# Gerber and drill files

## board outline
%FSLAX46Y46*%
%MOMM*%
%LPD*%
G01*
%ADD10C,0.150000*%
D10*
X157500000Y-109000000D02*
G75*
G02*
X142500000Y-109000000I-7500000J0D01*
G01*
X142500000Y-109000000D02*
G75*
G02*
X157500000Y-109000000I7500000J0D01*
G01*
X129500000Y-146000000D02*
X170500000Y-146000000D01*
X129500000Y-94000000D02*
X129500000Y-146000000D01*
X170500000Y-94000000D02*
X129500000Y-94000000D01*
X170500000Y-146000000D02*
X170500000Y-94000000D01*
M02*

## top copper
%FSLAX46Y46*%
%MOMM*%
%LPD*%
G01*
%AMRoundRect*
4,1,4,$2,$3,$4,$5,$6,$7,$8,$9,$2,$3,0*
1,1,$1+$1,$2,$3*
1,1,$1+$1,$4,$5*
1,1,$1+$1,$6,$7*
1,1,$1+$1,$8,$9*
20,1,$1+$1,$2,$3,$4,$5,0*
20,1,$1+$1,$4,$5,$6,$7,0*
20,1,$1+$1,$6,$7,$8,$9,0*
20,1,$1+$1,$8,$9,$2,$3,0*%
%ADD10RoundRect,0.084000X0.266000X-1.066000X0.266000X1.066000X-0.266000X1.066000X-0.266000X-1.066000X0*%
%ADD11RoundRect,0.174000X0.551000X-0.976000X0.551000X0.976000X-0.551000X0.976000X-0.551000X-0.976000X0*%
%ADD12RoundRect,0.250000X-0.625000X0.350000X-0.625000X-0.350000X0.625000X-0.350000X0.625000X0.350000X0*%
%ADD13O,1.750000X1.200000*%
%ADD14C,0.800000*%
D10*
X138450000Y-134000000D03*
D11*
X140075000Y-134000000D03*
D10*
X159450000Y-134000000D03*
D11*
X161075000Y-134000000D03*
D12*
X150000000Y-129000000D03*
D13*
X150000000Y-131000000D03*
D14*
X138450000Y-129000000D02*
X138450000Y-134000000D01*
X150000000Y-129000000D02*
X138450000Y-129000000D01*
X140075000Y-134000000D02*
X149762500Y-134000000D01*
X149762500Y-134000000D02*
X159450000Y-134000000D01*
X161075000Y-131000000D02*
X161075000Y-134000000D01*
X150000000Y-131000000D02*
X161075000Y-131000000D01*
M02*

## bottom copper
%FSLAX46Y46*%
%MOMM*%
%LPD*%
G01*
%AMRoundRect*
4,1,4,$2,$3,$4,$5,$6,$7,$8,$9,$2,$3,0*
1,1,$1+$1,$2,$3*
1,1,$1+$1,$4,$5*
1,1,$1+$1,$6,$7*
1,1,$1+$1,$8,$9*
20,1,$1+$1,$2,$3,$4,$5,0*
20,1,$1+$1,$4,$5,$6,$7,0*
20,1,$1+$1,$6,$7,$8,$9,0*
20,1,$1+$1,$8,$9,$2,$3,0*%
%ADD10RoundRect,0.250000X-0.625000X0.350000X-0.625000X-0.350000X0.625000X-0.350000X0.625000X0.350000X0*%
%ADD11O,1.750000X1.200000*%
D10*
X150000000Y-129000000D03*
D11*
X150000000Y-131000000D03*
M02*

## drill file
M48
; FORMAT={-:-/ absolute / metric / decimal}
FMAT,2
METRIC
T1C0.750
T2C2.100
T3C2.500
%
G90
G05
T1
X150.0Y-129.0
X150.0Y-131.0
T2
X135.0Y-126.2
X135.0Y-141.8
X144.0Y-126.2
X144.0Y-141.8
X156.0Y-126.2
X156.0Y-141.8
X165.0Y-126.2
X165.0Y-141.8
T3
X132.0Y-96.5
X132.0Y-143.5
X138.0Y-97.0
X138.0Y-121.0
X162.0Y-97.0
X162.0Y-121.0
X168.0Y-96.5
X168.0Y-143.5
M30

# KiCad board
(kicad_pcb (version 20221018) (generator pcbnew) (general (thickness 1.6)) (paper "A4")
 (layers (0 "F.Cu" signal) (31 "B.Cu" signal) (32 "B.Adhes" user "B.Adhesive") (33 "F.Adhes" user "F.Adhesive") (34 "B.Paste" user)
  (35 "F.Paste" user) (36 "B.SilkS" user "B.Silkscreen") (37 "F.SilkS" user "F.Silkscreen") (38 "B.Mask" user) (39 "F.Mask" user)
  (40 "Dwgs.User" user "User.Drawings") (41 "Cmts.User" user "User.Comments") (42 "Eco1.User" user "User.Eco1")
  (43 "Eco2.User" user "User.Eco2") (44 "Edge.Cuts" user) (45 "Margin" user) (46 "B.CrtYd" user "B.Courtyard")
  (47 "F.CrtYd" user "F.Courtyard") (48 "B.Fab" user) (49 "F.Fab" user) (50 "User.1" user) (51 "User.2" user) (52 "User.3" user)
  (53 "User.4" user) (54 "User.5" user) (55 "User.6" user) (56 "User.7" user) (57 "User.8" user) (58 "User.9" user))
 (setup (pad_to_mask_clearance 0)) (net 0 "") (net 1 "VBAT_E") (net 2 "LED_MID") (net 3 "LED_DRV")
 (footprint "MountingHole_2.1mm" (layer "F.Cu") (at 144 126.2)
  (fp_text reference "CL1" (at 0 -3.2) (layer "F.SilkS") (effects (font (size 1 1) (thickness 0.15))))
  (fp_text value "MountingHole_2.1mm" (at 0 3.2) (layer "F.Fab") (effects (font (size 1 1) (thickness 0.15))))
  (pad "" np_thru_hole circle (at 0 0) (size 2.1 2.1) (drill 2.1) (layers "*.Cu" "*.Mask")))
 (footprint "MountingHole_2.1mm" (layer "F.Cu") (at 135 126.2)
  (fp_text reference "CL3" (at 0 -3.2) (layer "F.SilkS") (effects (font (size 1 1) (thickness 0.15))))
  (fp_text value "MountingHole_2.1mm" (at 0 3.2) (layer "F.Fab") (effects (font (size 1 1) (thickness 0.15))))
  (pad "" np_thru_hole circle (at 0 0) (size 2.1 2.1) (drill 2.1) (layers "*.Cu" "*.Mask")))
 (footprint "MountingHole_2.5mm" (layer "F.Cu") (at 138 121)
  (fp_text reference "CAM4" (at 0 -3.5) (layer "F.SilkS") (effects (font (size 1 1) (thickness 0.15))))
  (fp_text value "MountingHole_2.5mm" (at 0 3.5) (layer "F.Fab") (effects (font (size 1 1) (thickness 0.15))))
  (pad "" np_thru_hole circle (at 0 0) (size 2.5 2.5) (drill 2.5) (layers "*.Cu" "*.Mask")))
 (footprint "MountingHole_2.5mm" (layer "F.Cu") (at 168 96.5)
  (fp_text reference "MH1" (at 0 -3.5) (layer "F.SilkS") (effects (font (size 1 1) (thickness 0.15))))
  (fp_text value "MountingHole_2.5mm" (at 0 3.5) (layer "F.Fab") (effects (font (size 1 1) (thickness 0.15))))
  (pad "" np_thru_hole circle (at 0 0) (size 2.5 2.5) (drill 2.5) (layers "*.Cu" "*.Mask")))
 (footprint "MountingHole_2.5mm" (layer "F.Cu") (at 132 96.5)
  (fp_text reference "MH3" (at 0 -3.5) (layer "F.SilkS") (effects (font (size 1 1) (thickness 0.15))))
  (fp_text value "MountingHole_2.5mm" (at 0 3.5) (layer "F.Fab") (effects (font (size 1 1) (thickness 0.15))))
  (pad "" np_thru_hole circle (at 0 0) (size 2.5 2.5) (drill 2.5) (layers "*.Cu" "*.Mask")))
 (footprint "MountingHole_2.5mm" (layer "F.Cu") (at 138 97)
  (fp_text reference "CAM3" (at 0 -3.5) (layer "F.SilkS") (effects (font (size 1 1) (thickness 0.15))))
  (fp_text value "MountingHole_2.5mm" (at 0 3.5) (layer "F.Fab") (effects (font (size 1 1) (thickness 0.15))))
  (pad "" np_thru_hole circle (at 0 0) (size 2.5 2.5) (drill 2.5) (layers "*.Cu" "*.Mask")))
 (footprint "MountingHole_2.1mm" (layer "F.Cu") (at 135 141.8)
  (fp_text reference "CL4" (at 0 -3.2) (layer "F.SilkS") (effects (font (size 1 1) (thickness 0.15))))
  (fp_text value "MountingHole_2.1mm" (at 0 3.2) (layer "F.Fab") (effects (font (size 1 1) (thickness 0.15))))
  (pad "" np_thru_hole circle (at 0 0) (size 2.1 2.1) (drill 2.1) (layers "*.Cu" "*.Mask")))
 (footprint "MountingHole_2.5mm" (layer "F.Cu") (at 168 143.5)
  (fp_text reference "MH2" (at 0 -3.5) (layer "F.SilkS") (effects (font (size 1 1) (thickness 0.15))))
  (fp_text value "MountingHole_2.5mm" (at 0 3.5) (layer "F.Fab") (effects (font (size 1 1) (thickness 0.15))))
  (pad "" np_thru_hole circle (at 0 0) (size 2.5 2.5) (drill 2.5) (layers "*.Cu" "*.Mask")))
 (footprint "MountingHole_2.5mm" (layer "F.Cu") (at 162 121)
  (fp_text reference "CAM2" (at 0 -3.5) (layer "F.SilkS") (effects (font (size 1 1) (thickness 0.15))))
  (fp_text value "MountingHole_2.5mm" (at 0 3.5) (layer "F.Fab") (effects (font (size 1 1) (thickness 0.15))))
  (pad "" np_thru_hole circle (at 0 0) (size 2.5 2.5) (drill 2.5) (layers "*.Cu" "*.Mask")))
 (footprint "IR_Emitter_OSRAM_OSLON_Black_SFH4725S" (layer "F.Cu") (at 139.5 134 90)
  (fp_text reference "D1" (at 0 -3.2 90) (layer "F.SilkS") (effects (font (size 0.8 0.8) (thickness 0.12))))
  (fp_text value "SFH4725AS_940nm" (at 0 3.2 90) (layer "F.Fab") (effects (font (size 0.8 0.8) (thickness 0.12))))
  (pad "1" smd roundrect (at 0 -1.05 90) (size 2.3 0.7) (layers "F.Cu" "F.Paste" "F.Mask") (roundrect_rratio 0.12) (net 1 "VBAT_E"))
  (pad "2" smd roundrect (at 0 0.575 90) (size 2.3 1.45) (layers "F.Cu" "F.Paste" "F.Mask") (roundrect_rratio 0.12) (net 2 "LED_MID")))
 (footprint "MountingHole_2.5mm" (layer "F.Cu") (at 132 143.5)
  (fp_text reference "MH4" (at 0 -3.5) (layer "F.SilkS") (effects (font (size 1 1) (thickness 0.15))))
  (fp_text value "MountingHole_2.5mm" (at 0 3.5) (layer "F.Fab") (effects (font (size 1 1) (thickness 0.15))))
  (pad "" np_thru_hole circle (at 0 0) (size 2.5 2.5) (drill 2.5) (layers "*.Cu" "*.Mask")))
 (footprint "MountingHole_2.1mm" (layer "F.Cu") (at 156 141.8)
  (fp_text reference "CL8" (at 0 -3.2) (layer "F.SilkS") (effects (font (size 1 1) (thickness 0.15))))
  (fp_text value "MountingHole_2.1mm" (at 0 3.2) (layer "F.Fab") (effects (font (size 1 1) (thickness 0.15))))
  (pad "" np_thru_hole circle (at 0 0) (size 2.1 2.1) (drill 2.1) (layers "*.Cu" "*.Mask")))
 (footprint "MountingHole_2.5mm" (layer "F.Cu") (at 162 97)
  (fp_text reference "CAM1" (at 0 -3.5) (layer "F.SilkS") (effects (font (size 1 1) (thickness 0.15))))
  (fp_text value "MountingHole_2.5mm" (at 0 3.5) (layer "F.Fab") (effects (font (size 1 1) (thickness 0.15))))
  (pad "" np_thru_hole circle (at 0 0) (size 2.5 2.5) (drill 2.5) (layers "*.Cu" "*.Mask")))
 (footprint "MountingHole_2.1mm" (layer "F.Cu") (at 165 126.2)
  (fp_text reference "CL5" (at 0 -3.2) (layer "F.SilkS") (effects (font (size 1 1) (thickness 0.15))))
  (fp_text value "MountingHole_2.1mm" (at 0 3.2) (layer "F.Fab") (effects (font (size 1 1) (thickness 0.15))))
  (pad "" np_thru_hole circle (at 0 0) (size 2.1 2.1) (drill 2.1) (layers "*.Cu" "*.Mask")))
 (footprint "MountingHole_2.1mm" (layer "F.Cu") (at 156 126.2)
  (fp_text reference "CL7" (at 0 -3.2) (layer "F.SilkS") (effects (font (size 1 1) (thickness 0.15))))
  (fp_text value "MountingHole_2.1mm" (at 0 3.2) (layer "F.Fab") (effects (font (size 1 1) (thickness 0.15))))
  (pad "" np_thru_hole circle (at 0 0) (size 2.1 2.1) (drill 2.1) (layers "*.Cu" "*.Mask")))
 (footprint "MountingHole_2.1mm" (layer "F.Cu") (at 165 141.8)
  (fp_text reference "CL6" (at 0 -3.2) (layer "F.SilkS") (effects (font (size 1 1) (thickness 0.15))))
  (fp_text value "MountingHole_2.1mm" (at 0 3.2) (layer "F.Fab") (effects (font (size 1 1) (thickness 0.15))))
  (pad "" np_thru_hole circle (at 0 0) (size 2.1 2.1) (drill 2.1) (layers "*.Cu" "*.Mask")))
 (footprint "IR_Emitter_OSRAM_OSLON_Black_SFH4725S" (layer "F.Cu") (at 160.5 134 90)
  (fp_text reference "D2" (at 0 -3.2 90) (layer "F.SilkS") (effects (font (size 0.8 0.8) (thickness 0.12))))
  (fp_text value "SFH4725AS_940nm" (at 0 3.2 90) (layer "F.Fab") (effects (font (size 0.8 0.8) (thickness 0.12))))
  (pad "1" smd roundrect (at 0 -1.05 90) (size 2.3 0.7) (layers "F.Cu" "F.Paste" "F.Mask") (roundrect_rratio 0.12) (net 2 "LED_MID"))
  (pad "2" smd roundrect (at 0 0.575 90) (size 2.3 1.45) (layers "F.Cu" "F.Paste" "F.Mask") (roundrect_rratio 0.12) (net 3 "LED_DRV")))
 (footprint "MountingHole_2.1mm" (layer "F.Cu") (at 144 141.8)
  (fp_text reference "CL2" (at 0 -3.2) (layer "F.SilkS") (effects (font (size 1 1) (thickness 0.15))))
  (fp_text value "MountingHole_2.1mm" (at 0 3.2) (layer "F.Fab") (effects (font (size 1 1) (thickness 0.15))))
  (pad "" np_thru_hole circle (at 0 0) (size 2.1 2.1) (drill 2.1) (layers "*.Cu" "*.Mask")))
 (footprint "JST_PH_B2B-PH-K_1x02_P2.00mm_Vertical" (layer "B.Cu") (at 150 129 -90)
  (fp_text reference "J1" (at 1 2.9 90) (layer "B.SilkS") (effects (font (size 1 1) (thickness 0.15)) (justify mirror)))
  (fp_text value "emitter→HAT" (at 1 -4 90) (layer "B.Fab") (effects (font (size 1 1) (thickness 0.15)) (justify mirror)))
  (pad "1" thru_hole roundrect (at 0 0 270) (size 1.2 1.75) (drill 0.75) (layers "*.Cu" "*.Mask") (roundrect_rratio 0.208333)
   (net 1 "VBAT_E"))
  (pad "2" thru_hole oval (at 2 0 270) (size 1.2 1.75) (drill 0.75) (layers "*.Cu" "*.Mask") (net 3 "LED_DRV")))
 (gr_circle (center 150 109) (end 157.5 109) (stroke (width 0.15) (type default)) (fill none) (layer "Edge.Cuts"))
 (gr_line (start 129.5 146) (end 170.5 146) (stroke (width 0.15) (type default)) (layer "Edge.Cuts"))
 (gr_line (start 129.5 94) (end 129.5 146) (stroke (width 0.15) (type default)) (layer "Edge.Cuts"))
 (gr_line (start 170.5 94) (end 129.5 94) (stroke (width 0.15) (type default)) (layer "Edge.Cuts"))
 (gr_line (start 170.5 146) (end 170.5 94) (stroke (width 0.15) (type default)) (layer "Edge.Cuts"))
 (segment (start 138.45 129) (end 138.45 134) (width 0.8) (layer "F.Cu") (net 1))
 (segment (start 150 129) (end 138.45 129) (width 0.8) (layer "F.Cu") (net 1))
 (segment (start 140.075 134) (end 149.7625 134) (width 0.8) (layer "F.Cu") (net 2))
 (segment (start 149.7625 134) (end 159.45 134) (width 0.8) (layer "F.Cu") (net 2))
 (segment (start 161.075 131) (end 161.075 134) (width 0.8) (layer "F.Cu") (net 3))
 (segment (start 150 131) (end 161.075 131) (width 0.8) (layer "F.Cu") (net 3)))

